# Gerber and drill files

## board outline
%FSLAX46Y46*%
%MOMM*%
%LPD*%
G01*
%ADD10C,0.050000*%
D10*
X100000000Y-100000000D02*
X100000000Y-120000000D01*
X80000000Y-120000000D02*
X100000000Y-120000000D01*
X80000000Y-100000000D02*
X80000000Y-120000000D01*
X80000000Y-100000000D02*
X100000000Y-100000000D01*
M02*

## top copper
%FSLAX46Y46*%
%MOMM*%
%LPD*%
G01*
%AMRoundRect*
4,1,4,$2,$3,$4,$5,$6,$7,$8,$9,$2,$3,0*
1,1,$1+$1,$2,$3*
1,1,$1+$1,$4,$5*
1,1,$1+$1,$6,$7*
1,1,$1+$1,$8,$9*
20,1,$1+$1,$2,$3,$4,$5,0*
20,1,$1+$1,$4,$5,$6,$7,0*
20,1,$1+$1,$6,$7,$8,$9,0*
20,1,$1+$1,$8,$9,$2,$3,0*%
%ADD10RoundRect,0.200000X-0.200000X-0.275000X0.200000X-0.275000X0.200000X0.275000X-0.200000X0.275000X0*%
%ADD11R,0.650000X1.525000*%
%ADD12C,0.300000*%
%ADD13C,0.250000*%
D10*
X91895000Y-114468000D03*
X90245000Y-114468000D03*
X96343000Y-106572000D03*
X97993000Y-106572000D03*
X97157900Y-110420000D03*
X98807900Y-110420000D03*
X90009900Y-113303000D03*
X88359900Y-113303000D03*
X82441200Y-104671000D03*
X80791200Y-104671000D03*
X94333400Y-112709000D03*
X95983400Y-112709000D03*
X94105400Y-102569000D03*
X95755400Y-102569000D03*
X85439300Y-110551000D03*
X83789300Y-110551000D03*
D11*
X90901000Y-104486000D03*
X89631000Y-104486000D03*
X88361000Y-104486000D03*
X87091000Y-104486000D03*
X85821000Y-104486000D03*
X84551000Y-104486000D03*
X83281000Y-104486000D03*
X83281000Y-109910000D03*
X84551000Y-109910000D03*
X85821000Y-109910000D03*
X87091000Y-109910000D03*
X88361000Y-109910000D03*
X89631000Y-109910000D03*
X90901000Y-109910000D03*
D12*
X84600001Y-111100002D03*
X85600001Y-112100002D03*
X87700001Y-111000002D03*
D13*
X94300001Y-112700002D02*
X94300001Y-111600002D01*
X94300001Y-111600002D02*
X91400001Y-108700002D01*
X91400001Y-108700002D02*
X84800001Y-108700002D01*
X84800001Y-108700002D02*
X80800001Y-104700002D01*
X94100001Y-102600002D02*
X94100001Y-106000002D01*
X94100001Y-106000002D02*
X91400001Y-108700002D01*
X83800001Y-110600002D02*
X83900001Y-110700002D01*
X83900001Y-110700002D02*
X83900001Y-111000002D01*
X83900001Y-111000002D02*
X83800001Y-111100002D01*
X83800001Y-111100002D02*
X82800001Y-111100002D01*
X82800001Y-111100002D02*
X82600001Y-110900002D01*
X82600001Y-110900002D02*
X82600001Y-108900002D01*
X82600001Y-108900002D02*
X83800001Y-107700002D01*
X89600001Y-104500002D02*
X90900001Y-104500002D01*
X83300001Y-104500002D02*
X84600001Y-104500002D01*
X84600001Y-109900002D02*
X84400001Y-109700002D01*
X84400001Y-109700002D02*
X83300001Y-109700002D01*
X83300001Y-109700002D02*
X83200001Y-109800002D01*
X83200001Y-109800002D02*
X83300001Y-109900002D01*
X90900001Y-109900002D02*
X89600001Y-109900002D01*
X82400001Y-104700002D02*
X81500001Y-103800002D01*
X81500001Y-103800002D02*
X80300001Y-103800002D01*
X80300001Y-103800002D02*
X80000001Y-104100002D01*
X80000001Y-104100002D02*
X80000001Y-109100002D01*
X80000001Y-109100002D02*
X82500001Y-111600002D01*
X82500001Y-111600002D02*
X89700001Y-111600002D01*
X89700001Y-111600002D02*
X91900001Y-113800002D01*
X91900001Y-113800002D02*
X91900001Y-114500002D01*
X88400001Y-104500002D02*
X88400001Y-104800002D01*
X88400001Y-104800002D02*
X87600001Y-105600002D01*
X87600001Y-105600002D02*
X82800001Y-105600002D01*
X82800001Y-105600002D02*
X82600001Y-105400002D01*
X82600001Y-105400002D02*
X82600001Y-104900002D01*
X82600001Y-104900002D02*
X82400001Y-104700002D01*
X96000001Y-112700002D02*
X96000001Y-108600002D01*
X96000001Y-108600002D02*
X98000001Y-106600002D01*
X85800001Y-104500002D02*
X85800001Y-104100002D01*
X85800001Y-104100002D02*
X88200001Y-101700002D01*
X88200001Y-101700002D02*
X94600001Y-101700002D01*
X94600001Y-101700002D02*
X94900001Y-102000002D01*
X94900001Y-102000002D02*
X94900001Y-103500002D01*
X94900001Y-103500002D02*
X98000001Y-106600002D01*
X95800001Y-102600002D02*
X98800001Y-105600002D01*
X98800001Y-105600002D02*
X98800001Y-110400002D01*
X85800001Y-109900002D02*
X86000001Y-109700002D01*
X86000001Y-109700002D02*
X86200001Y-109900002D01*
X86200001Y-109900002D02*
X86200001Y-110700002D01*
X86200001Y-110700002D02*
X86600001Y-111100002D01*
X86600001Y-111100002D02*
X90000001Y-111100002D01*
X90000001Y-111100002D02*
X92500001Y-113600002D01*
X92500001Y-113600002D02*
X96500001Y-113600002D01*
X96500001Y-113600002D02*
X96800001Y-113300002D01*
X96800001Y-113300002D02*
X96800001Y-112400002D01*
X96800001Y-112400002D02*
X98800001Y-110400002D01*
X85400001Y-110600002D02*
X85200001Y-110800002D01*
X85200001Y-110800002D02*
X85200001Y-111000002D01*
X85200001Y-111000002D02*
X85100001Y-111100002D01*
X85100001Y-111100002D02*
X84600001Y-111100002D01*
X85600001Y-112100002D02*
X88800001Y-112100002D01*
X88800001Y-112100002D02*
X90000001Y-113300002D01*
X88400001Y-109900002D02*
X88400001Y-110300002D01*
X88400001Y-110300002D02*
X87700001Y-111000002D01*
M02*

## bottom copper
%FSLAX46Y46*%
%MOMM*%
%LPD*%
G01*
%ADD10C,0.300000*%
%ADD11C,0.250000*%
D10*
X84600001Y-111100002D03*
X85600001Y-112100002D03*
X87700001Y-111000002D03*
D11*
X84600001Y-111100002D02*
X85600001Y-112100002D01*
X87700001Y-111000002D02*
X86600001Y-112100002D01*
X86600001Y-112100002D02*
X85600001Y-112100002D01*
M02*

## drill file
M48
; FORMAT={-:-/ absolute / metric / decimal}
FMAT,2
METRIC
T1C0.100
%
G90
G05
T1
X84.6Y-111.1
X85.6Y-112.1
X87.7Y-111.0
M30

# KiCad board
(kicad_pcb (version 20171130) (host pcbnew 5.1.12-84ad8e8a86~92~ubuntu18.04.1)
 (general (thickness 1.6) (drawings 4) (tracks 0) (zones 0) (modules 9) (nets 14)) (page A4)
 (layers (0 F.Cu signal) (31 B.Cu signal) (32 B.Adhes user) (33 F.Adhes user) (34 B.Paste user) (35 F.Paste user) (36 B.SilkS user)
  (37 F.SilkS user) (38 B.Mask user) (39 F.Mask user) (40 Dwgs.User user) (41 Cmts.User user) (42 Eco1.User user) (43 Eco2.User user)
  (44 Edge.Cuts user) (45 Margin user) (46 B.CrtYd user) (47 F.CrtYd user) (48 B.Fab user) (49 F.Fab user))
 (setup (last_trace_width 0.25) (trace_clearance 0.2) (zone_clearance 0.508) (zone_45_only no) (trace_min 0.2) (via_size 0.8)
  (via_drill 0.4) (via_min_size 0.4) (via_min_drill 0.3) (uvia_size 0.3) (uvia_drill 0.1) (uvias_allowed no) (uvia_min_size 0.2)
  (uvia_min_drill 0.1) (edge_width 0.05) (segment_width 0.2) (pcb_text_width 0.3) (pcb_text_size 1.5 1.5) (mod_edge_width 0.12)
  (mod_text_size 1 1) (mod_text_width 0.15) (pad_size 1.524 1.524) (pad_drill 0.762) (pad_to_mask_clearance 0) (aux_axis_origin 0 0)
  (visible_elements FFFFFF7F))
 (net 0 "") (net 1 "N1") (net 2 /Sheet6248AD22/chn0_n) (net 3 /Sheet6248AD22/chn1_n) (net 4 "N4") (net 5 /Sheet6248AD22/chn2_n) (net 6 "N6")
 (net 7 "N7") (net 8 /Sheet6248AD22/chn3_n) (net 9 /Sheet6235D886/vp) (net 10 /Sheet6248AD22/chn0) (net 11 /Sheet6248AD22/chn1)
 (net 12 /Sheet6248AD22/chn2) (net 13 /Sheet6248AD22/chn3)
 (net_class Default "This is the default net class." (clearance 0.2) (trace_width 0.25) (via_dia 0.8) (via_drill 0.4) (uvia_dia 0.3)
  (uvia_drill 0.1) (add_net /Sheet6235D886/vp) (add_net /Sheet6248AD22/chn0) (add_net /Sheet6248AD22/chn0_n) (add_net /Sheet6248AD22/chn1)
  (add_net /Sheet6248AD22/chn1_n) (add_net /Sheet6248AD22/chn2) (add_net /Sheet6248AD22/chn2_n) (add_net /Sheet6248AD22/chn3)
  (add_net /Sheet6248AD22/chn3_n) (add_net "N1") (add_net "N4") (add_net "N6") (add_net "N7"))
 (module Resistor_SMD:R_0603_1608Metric (layer F.Cu) (at 91.070000 114.468000)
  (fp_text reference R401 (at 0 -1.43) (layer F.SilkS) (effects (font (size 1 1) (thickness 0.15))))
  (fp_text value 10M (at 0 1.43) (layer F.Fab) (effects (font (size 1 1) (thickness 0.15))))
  (pad 2 smd roundrect (at 0.825 0) (size 0.8 0.95) (layers F.Cu F.Mask F.Paste) (roundrect_rratio 0.25) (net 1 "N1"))
  (pad 1 smd roundrect (at -0.825 0) (size 0.8 0.95) (layers F.Cu F.Mask F.Paste) (roundrect_rratio 0.25) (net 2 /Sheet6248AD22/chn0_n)))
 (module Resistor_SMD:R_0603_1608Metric (layer F.Cu) (at 97.168000 106.572000)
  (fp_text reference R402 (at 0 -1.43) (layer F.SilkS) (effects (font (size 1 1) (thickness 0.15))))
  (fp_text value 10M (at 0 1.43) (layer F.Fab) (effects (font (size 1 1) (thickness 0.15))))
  (pad 1 smd roundrect (at -0.825 0) (size 0.8 0.95) (layers F.Cu F.Mask F.Paste) (roundrect_rratio 0.25) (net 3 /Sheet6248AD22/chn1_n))
  (pad 2 smd roundrect (at 0.825 0) (size 0.8 0.95) (layers F.Cu F.Mask F.Paste) (roundrect_rratio 0.25) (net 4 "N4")))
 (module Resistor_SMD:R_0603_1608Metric (layer F.Cu) (at 97.982900 110.420000)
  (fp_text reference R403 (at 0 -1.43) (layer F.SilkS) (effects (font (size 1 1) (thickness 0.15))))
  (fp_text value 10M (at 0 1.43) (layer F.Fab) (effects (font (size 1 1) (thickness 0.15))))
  (pad 1 smd roundrect (at -0.825 0) (size 0.8 0.95) (layers F.Cu F.Mask F.Paste) (roundrect_rratio 0.25) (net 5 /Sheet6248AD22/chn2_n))
  (pad 2 smd roundrect (at 0.825 0) (size 0.8 0.95) (layers F.Cu F.Mask F.Paste) (roundrect_rratio 0.25) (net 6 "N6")))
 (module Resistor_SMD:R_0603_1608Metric (layer F.Cu) (at 89.184900 113.303000)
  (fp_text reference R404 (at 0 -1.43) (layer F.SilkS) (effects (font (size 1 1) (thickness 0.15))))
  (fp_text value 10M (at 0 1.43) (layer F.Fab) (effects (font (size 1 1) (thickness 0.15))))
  (pad 2 smd roundrect (at 0.825 0) (size 0.8 0.95) (layers F.Cu F.Mask F.Paste) (roundrect_rratio 0.25) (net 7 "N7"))
  (pad 1 smd roundrect (at -0.825 0) (size 0.8 0.95) (layers F.Cu F.Mask F.Paste) (roundrect_rratio 0.25) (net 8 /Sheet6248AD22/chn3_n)))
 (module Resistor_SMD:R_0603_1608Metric (layer F.Cu) (at 81.616200 104.671000)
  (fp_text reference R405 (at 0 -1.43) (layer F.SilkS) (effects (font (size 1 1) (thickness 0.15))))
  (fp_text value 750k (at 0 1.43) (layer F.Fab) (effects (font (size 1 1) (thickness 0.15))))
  (pad 2 smd roundrect (at 0.825 0) (size 0.8 0.95) (layers F.Cu F.Mask F.Paste) (roundrect_rratio 0.25) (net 1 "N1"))
  (pad 1 smd roundrect (at -0.825 0) (size 0.8 0.95) (layers F.Cu F.Mask F.Paste) (roundrect_rratio 0.25) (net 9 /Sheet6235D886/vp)))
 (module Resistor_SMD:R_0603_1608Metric (layer F.Cu) (at 95.158400 112.709000)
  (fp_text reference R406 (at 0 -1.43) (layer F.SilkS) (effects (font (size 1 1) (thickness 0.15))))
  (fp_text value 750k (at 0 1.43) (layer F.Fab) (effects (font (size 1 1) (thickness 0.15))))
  (pad 1 smd roundrect (at -0.825 0) (size 0.8 0.95) (layers F.Cu F.Mask F.Paste) (roundrect_rratio 0.25) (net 9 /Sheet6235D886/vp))
  (pad 2 smd roundrect (at 0.825 0) (size 0.8 0.95) (layers F.Cu F.Mask F.Paste) (roundrect_rratio 0.25) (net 4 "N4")))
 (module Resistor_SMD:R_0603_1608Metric (layer F.Cu) (at 94.930400 102.569000)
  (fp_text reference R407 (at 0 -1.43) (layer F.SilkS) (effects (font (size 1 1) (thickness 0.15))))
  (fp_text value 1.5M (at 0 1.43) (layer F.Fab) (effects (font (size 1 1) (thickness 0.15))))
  (pad 1 smd roundrect (at -0.825 0) (size 0.8 0.95) (layers F.Cu F.Mask F.Paste) (roundrect_rratio 0.25) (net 9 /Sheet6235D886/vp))
  (pad 2 smd roundrect (at 0.825 0) (size 0.8 0.95) (layers F.Cu F.Mask F.Paste) (roundrect_rratio 0.25) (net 6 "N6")))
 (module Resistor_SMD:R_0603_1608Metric (layer F.Cu) (at 84.614300 110.551000)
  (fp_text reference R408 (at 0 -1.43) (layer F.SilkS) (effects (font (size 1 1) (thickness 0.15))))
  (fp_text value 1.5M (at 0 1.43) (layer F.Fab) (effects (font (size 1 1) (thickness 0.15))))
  (pad 2 smd roundrect (at 0.825 0) (size 0.8 0.95) (layers F.Cu F.Mask F.Paste) (roundrect_rratio 0.25) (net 7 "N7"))
  (pad 1 smd roundrect (at -0.825 0) (size 0.8 0.95) (layers F.Cu F.Mask F.Paste) (roundrect_rratio 0.25) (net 9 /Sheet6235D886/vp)))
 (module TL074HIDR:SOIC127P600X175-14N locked (layer F.Cu) (at 87.091000 107.198000 270.000000)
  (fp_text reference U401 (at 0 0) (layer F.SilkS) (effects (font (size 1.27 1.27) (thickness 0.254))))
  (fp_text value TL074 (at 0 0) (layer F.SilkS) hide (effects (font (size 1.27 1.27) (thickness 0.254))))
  (pad 1 smd rect (at -2.712 -3.81) (size 0.65 1.525) (layers F.Cu F.Mask F.Paste) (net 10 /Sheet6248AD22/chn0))
  (pad 2 smd rect (at -2.712 -2.54) (size 0.65 1.525) (layers F.Cu F.Mask F.Paste) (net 10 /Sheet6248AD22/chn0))
  (pad 3 smd rect (at -2.712 -1.27) (size 0.65 1.525) (layers F.Cu F.Mask F.Paste) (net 1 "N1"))
  (pad 4 smd rect (at -2.712 0) (size 0.65 1.525) (layers F.Cu F.Mask F.Paste))
  (pad 5 smd rect (at -2.712 1.27) (size 0.65 1.525) (layers F.Cu F.Mask F.Paste) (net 4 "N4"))
  (pad 6 smd rect (at -2.712 2.54) (size 0.65 1.525) (layers F.Cu F.Mask F.Paste) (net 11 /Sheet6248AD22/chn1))
  (pad 7 smd rect (at -2.712 3.81) (size 0.65 1.525) (layers F.Cu F.Mask F.Paste) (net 11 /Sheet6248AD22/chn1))
  (pad 8 smd rect (at 2.712 3.81) (size 0.65 1.525) (layers F.Cu F.Mask F.Paste) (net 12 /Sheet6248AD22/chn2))
  (pad 9 smd rect (at 2.712 2.54) (size 0.65 1.525) (layers F.Cu F.Mask F.Paste) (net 12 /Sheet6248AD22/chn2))
  (pad 10 smd rect (at 2.712 1.27) (size 0.65 1.525) (layers F.Cu F.Mask F.Paste) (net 6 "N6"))
  (pad 11 smd rect (at 2.712 0) (size 0.65 1.525) (layers F.Cu F.Mask F.Paste))
  (pad 12 smd rect (at 2.712 -1.27) (size 0.65 1.525) (layers F.Cu F.Mask F.Paste) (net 7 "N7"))
  (pad 13 smd rect (at 2.712 -2.54) (size 0.65 1.525) (layers F.Cu F.Mask F.Paste) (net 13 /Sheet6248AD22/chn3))
  (pad 14 smd rect (at 2.712 -3.81) (size 0.65 1.525) (layers F.Cu F.Mask F.Paste) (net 13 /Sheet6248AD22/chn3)))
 (gr_line (start 100 100) (end 100 120) (layer Edge.Cuts) (width 0.05))
 (gr_line (start 80 120) (end 100 120) (layer Edge.Cuts) (width 0.05))
 (gr_line (start 80 100) (end 80 120) (layer Edge.Cuts) (width 0.05))
 (gr_line (start 80 100) (end 100 100) (layer Edge.Cuts) (width 0.05))
 (segment (start 94.300001 112.700002) (end 94.300001 111.600002) (width 0.250000) (layer F.Cu) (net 9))
 (segment (start 94.300001 111.600002) (end 91.400001 108.700002) (width 0.250000) (layer F.Cu) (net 9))
 (segment (start 91.400001 108.700002) (end 84.800001 108.700002) (width 0.250000) (layer F.Cu) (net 9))
 (segment (start 84.800001 108.700002) (end 80.800001 104.700002) (width 0.250000) (layer F.Cu) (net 9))
 (segment (start 94.100001 102.600002) (end 94.100001 106.000002) (width 0.250000) (layer F.Cu) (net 9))
 (segment (start 94.100001 106.000002) (end 91.400001 108.700002) (width 0.250000) (layer F.Cu) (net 9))
 (segment (start 83.800001 110.600002) (end 83.900001 110.700002) (width 0.250000) (layer F.Cu) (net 9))
 (segment (start 83.900001 110.700002) (end 83.900001 111.000002) (width 0.250000) (layer F.Cu) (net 9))
 (segment (start 83.900001 111.000002) (end 83.800001 111.100002) (width 0.250000) (layer F.Cu) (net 9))
 (segment (start 83.800001 111.100002) (end 82.800001 111.100002) (width 0.250000) (layer F.Cu) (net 9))
 (segment (start 82.800001 111.100002) (end 82.600001 110.900002) (width 0.250000) (layer F.Cu) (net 9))
 (segment (start 82.600001 110.900002) (end 82.600001 108.900002) (width 0.250000) (layer F.Cu) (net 9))
 (segment (start 82.600001 108.900002) (end 83.800001 107.700002) (width 0.250000) (layer F.Cu) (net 9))
 (segment (start 89.600001 104.500002) (end 90.900001 104.500002) (width 0.250000) (layer F.Cu) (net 10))
 (segment (start 83.300001 104.500002) (end 84.600001 104.500002) (width 0.250000) (layer F.Cu) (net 11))
 (segment (start 84.600001 109.900002) (end 84.400001 109.700002) (width 0.250000) (layer F.Cu) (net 12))
 (segment (start 84.400001 109.700002) (end 83.300001 109.700002) (width 0.250000) (layer F.Cu) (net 12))
 (segment (start 83.300001 109.700002) (end 83.200001 109.800002) (width 0.250000) (layer F.Cu) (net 12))
 (segment (start 83.200001 109.800002) (end 83.300001 109.900002) (width 0.250000) (layer F.Cu) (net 12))
 (segment (start 90.900001 109.900002) (end 89.600001 109.900002) (width 0.250000) (layer F.Cu) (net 13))
 (segment (start 82.400001 104.700002) (end 81.500001 103.800002) (width 0.250000) (layer F.Cu) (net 1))
 (segment (start 81.500001 103.800002) (end 80.300001 103.800002) (width 0.250000) (layer F.Cu) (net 1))
 (segment (start 80.300001 103.800002) (end 80.000001 104.100002) (width 0.250000) (layer F.Cu) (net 1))
 (segment (start 80.000001 104.100002) (end 80.000001 109.100002) (width 0.250000) (layer F.Cu) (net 1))
 (segment (start 80.000001 109.100002) (end 82.500001 111.600002) (width 0.250000) (layer F.Cu) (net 1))
 (segment (start 82.500001 111.600002) (end 89.700001 111.600002) (width 0.250000) (layer F.Cu) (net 1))
 (segment (start 89.700001 111.600002) (end 91.900001 113.800002) (width 0.250000) (layer F.Cu) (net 1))
 (segment (start 91.900001 113.800002) (end 91.900001 114.500002) (width 0.250000) (layer F.Cu) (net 1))
 (segment (start 88.400001 104.500002) (end 88.400001 104.800002) (width 0.250000) (layer F.Cu) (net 1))
 (segment (start 88.400001 104.800002) (end 87.600001 105.600002) (width 0.250000) (layer F.Cu) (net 1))
 (segment (start 87.600001 105.600002) (end 82.800001 105.600002) (width 0.250000) (layer F.Cu) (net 1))
 (segment (start 82.800001 105.600002) (end 82.600001 105.400002) (width 0.250000) (layer F.Cu) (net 1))
 (segment (start 82.600001 105.400002) (end 82.600001 104.900002) (width 0.250000) (layer F.Cu) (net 1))
 (segment (start 82.600001 104.900002) (end 82.400001 104.700002) (width 0.250000) (layer F.Cu) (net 1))
 (segment (start 96.000001 112.700002) (end 96.000001 108.600002) (width 0.250000) (layer F.Cu) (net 4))
 (segment (start 96.000001 108.600002) (end 98.000001 106.600002) (width 0.250000) (layer F.Cu) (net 4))
 (segment (start 85.800001 104.500002) (end 85.800001 104.100002) (width 0.250000) (layer F.Cu) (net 4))
 (segment (start 85.800001 104.100002) (end 88.200001 101.700002) (width 0.250000) (layer F.Cu) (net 4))
 (segment (start 88.200001 101.700002) (end 94.600001 101.700002) (width 0.250000) (layer F.Cu) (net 4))
 (segment (start 94.600001 101.700002) (end 94.900001 102.000002) (width 0.250000) (layer F.Cu) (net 4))
 (segment (start 94.900001 102.000002) (end 94.900001 103.500002) (width 0.250000) (layer F.Cu) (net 4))
 (segment (start 94.900001 103.500002) (end 98.000001 106.600002) (width 0.250000) (layer F.Cu) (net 4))
 (segment (start 95.800001 102.600002) (end 98.800001 105.600002) (width 0.250000) (layer F.Cu) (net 6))
 (segment (start 98.800001 105.600002) (end 98.800001 110.400002) (width 0.250000) (layer F.Cu) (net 6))
 (segment (start 85.800001 109.900002) (end 86.000001 109.700002) (width 0.250000) (layer F.Cu) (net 6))
 (segment (start 86.000001 109.700002) (end 86.200001 109.900002) (width 0.250000) (layer F.Cu) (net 6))
 (segment (start 86.200001 109.900002) (end 86.200001 110.700002) (width 0.250000) (layer F.Cu) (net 6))
 (segment (start 86.200001 110.700002) (end 86.600001 111.100002) (width 0.250000) (layer F.Cu) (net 6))
 (segment (start 86.600001 111.100002) (end 90.000001 111.100002) (width 0.250000) (layer F.Cu) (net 6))
 (segment (start 90.000001 111.100002) (end 92.500001 113.600002) (width 0.250000) (layer F.Cu) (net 6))
 (segment (start 92.500001 113.600002) (end 96.500001 113.600002) (width 0.250000) (layer F.Cu) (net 6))
 (segment (start 96.500001 113.600002) (end 96.800001 113.300002) (width 0.250000) (layer F.Cu) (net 6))
 (segment (start 96.800001 113.300002) (end 96.800001 112.400002) (width 0.250000) (layer F.Cu) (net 6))
 (segment (start 96.800001 112.400002) (end 98.800001 110.400002) (width 0.250000) (layer F.Cu) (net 6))
 (segment (start 85.400001 110.600002) (end 85.200001 110.800002) (width 0.250000) (layer F.Cu) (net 7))
 (segment (start 85.200001 110.800002) (end 85.200001 111.000002) (width 0.250000) (layer F.Cu) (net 7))
 (segment (start 85.200001 111.000002) (end 85.100001 111.100002) (width 0.250000) (layer F.Cu) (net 7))
 (segment (start 85.100001 111.100002) (end 84.600001 111.100002) (width 0.250000) (layer F.Cu) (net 7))
 (segment (start 84.600001 111.100002) (end 85.600001 112.100002) (width 0.250000) (layer B.Cu) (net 7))
 (segment (start 85.600001 112.100002) (end 88.800001 112.100002) (width 0.250000) (layer F.Cu) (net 7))
 (segment (start 88.800001 112.100002) (end 90.000001 113.300002) (width 0.250000) (layer F.Cu) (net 7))
 (segment (start 88.400001 109.900002) (end 88.400001 110.300002) (width 0.250000) (layer F.Cu) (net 7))
 (segment (start 88.400001 110.300002) (end 87.700001 111.000002) (width 0.250000) (layer F.Cu) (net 7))
 (segment (start 87.700001 111.000002) (end 86.600001 112.100002) (width 0.250000) (layer B.Cu) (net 7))
 (segment (start 86.600001 112.100002) (end 85.600001 112.100002) (width 0.250000) (layer B.Cu) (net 7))
 (via micro (at 84.600001 111.100002) (size 0.300000) (drill 0.100000) (layers F.Cu B.Cu) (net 7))
 (via micro (at 85.600001 112.100002) (size 0.300000) (drill 0.100000) (layers F.Cu B.Cu) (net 7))
 (via micro (at 87.700001 111.000002) (size 0.300000) (drill 0.100000) (layers F.Cu B.Cu) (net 7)))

